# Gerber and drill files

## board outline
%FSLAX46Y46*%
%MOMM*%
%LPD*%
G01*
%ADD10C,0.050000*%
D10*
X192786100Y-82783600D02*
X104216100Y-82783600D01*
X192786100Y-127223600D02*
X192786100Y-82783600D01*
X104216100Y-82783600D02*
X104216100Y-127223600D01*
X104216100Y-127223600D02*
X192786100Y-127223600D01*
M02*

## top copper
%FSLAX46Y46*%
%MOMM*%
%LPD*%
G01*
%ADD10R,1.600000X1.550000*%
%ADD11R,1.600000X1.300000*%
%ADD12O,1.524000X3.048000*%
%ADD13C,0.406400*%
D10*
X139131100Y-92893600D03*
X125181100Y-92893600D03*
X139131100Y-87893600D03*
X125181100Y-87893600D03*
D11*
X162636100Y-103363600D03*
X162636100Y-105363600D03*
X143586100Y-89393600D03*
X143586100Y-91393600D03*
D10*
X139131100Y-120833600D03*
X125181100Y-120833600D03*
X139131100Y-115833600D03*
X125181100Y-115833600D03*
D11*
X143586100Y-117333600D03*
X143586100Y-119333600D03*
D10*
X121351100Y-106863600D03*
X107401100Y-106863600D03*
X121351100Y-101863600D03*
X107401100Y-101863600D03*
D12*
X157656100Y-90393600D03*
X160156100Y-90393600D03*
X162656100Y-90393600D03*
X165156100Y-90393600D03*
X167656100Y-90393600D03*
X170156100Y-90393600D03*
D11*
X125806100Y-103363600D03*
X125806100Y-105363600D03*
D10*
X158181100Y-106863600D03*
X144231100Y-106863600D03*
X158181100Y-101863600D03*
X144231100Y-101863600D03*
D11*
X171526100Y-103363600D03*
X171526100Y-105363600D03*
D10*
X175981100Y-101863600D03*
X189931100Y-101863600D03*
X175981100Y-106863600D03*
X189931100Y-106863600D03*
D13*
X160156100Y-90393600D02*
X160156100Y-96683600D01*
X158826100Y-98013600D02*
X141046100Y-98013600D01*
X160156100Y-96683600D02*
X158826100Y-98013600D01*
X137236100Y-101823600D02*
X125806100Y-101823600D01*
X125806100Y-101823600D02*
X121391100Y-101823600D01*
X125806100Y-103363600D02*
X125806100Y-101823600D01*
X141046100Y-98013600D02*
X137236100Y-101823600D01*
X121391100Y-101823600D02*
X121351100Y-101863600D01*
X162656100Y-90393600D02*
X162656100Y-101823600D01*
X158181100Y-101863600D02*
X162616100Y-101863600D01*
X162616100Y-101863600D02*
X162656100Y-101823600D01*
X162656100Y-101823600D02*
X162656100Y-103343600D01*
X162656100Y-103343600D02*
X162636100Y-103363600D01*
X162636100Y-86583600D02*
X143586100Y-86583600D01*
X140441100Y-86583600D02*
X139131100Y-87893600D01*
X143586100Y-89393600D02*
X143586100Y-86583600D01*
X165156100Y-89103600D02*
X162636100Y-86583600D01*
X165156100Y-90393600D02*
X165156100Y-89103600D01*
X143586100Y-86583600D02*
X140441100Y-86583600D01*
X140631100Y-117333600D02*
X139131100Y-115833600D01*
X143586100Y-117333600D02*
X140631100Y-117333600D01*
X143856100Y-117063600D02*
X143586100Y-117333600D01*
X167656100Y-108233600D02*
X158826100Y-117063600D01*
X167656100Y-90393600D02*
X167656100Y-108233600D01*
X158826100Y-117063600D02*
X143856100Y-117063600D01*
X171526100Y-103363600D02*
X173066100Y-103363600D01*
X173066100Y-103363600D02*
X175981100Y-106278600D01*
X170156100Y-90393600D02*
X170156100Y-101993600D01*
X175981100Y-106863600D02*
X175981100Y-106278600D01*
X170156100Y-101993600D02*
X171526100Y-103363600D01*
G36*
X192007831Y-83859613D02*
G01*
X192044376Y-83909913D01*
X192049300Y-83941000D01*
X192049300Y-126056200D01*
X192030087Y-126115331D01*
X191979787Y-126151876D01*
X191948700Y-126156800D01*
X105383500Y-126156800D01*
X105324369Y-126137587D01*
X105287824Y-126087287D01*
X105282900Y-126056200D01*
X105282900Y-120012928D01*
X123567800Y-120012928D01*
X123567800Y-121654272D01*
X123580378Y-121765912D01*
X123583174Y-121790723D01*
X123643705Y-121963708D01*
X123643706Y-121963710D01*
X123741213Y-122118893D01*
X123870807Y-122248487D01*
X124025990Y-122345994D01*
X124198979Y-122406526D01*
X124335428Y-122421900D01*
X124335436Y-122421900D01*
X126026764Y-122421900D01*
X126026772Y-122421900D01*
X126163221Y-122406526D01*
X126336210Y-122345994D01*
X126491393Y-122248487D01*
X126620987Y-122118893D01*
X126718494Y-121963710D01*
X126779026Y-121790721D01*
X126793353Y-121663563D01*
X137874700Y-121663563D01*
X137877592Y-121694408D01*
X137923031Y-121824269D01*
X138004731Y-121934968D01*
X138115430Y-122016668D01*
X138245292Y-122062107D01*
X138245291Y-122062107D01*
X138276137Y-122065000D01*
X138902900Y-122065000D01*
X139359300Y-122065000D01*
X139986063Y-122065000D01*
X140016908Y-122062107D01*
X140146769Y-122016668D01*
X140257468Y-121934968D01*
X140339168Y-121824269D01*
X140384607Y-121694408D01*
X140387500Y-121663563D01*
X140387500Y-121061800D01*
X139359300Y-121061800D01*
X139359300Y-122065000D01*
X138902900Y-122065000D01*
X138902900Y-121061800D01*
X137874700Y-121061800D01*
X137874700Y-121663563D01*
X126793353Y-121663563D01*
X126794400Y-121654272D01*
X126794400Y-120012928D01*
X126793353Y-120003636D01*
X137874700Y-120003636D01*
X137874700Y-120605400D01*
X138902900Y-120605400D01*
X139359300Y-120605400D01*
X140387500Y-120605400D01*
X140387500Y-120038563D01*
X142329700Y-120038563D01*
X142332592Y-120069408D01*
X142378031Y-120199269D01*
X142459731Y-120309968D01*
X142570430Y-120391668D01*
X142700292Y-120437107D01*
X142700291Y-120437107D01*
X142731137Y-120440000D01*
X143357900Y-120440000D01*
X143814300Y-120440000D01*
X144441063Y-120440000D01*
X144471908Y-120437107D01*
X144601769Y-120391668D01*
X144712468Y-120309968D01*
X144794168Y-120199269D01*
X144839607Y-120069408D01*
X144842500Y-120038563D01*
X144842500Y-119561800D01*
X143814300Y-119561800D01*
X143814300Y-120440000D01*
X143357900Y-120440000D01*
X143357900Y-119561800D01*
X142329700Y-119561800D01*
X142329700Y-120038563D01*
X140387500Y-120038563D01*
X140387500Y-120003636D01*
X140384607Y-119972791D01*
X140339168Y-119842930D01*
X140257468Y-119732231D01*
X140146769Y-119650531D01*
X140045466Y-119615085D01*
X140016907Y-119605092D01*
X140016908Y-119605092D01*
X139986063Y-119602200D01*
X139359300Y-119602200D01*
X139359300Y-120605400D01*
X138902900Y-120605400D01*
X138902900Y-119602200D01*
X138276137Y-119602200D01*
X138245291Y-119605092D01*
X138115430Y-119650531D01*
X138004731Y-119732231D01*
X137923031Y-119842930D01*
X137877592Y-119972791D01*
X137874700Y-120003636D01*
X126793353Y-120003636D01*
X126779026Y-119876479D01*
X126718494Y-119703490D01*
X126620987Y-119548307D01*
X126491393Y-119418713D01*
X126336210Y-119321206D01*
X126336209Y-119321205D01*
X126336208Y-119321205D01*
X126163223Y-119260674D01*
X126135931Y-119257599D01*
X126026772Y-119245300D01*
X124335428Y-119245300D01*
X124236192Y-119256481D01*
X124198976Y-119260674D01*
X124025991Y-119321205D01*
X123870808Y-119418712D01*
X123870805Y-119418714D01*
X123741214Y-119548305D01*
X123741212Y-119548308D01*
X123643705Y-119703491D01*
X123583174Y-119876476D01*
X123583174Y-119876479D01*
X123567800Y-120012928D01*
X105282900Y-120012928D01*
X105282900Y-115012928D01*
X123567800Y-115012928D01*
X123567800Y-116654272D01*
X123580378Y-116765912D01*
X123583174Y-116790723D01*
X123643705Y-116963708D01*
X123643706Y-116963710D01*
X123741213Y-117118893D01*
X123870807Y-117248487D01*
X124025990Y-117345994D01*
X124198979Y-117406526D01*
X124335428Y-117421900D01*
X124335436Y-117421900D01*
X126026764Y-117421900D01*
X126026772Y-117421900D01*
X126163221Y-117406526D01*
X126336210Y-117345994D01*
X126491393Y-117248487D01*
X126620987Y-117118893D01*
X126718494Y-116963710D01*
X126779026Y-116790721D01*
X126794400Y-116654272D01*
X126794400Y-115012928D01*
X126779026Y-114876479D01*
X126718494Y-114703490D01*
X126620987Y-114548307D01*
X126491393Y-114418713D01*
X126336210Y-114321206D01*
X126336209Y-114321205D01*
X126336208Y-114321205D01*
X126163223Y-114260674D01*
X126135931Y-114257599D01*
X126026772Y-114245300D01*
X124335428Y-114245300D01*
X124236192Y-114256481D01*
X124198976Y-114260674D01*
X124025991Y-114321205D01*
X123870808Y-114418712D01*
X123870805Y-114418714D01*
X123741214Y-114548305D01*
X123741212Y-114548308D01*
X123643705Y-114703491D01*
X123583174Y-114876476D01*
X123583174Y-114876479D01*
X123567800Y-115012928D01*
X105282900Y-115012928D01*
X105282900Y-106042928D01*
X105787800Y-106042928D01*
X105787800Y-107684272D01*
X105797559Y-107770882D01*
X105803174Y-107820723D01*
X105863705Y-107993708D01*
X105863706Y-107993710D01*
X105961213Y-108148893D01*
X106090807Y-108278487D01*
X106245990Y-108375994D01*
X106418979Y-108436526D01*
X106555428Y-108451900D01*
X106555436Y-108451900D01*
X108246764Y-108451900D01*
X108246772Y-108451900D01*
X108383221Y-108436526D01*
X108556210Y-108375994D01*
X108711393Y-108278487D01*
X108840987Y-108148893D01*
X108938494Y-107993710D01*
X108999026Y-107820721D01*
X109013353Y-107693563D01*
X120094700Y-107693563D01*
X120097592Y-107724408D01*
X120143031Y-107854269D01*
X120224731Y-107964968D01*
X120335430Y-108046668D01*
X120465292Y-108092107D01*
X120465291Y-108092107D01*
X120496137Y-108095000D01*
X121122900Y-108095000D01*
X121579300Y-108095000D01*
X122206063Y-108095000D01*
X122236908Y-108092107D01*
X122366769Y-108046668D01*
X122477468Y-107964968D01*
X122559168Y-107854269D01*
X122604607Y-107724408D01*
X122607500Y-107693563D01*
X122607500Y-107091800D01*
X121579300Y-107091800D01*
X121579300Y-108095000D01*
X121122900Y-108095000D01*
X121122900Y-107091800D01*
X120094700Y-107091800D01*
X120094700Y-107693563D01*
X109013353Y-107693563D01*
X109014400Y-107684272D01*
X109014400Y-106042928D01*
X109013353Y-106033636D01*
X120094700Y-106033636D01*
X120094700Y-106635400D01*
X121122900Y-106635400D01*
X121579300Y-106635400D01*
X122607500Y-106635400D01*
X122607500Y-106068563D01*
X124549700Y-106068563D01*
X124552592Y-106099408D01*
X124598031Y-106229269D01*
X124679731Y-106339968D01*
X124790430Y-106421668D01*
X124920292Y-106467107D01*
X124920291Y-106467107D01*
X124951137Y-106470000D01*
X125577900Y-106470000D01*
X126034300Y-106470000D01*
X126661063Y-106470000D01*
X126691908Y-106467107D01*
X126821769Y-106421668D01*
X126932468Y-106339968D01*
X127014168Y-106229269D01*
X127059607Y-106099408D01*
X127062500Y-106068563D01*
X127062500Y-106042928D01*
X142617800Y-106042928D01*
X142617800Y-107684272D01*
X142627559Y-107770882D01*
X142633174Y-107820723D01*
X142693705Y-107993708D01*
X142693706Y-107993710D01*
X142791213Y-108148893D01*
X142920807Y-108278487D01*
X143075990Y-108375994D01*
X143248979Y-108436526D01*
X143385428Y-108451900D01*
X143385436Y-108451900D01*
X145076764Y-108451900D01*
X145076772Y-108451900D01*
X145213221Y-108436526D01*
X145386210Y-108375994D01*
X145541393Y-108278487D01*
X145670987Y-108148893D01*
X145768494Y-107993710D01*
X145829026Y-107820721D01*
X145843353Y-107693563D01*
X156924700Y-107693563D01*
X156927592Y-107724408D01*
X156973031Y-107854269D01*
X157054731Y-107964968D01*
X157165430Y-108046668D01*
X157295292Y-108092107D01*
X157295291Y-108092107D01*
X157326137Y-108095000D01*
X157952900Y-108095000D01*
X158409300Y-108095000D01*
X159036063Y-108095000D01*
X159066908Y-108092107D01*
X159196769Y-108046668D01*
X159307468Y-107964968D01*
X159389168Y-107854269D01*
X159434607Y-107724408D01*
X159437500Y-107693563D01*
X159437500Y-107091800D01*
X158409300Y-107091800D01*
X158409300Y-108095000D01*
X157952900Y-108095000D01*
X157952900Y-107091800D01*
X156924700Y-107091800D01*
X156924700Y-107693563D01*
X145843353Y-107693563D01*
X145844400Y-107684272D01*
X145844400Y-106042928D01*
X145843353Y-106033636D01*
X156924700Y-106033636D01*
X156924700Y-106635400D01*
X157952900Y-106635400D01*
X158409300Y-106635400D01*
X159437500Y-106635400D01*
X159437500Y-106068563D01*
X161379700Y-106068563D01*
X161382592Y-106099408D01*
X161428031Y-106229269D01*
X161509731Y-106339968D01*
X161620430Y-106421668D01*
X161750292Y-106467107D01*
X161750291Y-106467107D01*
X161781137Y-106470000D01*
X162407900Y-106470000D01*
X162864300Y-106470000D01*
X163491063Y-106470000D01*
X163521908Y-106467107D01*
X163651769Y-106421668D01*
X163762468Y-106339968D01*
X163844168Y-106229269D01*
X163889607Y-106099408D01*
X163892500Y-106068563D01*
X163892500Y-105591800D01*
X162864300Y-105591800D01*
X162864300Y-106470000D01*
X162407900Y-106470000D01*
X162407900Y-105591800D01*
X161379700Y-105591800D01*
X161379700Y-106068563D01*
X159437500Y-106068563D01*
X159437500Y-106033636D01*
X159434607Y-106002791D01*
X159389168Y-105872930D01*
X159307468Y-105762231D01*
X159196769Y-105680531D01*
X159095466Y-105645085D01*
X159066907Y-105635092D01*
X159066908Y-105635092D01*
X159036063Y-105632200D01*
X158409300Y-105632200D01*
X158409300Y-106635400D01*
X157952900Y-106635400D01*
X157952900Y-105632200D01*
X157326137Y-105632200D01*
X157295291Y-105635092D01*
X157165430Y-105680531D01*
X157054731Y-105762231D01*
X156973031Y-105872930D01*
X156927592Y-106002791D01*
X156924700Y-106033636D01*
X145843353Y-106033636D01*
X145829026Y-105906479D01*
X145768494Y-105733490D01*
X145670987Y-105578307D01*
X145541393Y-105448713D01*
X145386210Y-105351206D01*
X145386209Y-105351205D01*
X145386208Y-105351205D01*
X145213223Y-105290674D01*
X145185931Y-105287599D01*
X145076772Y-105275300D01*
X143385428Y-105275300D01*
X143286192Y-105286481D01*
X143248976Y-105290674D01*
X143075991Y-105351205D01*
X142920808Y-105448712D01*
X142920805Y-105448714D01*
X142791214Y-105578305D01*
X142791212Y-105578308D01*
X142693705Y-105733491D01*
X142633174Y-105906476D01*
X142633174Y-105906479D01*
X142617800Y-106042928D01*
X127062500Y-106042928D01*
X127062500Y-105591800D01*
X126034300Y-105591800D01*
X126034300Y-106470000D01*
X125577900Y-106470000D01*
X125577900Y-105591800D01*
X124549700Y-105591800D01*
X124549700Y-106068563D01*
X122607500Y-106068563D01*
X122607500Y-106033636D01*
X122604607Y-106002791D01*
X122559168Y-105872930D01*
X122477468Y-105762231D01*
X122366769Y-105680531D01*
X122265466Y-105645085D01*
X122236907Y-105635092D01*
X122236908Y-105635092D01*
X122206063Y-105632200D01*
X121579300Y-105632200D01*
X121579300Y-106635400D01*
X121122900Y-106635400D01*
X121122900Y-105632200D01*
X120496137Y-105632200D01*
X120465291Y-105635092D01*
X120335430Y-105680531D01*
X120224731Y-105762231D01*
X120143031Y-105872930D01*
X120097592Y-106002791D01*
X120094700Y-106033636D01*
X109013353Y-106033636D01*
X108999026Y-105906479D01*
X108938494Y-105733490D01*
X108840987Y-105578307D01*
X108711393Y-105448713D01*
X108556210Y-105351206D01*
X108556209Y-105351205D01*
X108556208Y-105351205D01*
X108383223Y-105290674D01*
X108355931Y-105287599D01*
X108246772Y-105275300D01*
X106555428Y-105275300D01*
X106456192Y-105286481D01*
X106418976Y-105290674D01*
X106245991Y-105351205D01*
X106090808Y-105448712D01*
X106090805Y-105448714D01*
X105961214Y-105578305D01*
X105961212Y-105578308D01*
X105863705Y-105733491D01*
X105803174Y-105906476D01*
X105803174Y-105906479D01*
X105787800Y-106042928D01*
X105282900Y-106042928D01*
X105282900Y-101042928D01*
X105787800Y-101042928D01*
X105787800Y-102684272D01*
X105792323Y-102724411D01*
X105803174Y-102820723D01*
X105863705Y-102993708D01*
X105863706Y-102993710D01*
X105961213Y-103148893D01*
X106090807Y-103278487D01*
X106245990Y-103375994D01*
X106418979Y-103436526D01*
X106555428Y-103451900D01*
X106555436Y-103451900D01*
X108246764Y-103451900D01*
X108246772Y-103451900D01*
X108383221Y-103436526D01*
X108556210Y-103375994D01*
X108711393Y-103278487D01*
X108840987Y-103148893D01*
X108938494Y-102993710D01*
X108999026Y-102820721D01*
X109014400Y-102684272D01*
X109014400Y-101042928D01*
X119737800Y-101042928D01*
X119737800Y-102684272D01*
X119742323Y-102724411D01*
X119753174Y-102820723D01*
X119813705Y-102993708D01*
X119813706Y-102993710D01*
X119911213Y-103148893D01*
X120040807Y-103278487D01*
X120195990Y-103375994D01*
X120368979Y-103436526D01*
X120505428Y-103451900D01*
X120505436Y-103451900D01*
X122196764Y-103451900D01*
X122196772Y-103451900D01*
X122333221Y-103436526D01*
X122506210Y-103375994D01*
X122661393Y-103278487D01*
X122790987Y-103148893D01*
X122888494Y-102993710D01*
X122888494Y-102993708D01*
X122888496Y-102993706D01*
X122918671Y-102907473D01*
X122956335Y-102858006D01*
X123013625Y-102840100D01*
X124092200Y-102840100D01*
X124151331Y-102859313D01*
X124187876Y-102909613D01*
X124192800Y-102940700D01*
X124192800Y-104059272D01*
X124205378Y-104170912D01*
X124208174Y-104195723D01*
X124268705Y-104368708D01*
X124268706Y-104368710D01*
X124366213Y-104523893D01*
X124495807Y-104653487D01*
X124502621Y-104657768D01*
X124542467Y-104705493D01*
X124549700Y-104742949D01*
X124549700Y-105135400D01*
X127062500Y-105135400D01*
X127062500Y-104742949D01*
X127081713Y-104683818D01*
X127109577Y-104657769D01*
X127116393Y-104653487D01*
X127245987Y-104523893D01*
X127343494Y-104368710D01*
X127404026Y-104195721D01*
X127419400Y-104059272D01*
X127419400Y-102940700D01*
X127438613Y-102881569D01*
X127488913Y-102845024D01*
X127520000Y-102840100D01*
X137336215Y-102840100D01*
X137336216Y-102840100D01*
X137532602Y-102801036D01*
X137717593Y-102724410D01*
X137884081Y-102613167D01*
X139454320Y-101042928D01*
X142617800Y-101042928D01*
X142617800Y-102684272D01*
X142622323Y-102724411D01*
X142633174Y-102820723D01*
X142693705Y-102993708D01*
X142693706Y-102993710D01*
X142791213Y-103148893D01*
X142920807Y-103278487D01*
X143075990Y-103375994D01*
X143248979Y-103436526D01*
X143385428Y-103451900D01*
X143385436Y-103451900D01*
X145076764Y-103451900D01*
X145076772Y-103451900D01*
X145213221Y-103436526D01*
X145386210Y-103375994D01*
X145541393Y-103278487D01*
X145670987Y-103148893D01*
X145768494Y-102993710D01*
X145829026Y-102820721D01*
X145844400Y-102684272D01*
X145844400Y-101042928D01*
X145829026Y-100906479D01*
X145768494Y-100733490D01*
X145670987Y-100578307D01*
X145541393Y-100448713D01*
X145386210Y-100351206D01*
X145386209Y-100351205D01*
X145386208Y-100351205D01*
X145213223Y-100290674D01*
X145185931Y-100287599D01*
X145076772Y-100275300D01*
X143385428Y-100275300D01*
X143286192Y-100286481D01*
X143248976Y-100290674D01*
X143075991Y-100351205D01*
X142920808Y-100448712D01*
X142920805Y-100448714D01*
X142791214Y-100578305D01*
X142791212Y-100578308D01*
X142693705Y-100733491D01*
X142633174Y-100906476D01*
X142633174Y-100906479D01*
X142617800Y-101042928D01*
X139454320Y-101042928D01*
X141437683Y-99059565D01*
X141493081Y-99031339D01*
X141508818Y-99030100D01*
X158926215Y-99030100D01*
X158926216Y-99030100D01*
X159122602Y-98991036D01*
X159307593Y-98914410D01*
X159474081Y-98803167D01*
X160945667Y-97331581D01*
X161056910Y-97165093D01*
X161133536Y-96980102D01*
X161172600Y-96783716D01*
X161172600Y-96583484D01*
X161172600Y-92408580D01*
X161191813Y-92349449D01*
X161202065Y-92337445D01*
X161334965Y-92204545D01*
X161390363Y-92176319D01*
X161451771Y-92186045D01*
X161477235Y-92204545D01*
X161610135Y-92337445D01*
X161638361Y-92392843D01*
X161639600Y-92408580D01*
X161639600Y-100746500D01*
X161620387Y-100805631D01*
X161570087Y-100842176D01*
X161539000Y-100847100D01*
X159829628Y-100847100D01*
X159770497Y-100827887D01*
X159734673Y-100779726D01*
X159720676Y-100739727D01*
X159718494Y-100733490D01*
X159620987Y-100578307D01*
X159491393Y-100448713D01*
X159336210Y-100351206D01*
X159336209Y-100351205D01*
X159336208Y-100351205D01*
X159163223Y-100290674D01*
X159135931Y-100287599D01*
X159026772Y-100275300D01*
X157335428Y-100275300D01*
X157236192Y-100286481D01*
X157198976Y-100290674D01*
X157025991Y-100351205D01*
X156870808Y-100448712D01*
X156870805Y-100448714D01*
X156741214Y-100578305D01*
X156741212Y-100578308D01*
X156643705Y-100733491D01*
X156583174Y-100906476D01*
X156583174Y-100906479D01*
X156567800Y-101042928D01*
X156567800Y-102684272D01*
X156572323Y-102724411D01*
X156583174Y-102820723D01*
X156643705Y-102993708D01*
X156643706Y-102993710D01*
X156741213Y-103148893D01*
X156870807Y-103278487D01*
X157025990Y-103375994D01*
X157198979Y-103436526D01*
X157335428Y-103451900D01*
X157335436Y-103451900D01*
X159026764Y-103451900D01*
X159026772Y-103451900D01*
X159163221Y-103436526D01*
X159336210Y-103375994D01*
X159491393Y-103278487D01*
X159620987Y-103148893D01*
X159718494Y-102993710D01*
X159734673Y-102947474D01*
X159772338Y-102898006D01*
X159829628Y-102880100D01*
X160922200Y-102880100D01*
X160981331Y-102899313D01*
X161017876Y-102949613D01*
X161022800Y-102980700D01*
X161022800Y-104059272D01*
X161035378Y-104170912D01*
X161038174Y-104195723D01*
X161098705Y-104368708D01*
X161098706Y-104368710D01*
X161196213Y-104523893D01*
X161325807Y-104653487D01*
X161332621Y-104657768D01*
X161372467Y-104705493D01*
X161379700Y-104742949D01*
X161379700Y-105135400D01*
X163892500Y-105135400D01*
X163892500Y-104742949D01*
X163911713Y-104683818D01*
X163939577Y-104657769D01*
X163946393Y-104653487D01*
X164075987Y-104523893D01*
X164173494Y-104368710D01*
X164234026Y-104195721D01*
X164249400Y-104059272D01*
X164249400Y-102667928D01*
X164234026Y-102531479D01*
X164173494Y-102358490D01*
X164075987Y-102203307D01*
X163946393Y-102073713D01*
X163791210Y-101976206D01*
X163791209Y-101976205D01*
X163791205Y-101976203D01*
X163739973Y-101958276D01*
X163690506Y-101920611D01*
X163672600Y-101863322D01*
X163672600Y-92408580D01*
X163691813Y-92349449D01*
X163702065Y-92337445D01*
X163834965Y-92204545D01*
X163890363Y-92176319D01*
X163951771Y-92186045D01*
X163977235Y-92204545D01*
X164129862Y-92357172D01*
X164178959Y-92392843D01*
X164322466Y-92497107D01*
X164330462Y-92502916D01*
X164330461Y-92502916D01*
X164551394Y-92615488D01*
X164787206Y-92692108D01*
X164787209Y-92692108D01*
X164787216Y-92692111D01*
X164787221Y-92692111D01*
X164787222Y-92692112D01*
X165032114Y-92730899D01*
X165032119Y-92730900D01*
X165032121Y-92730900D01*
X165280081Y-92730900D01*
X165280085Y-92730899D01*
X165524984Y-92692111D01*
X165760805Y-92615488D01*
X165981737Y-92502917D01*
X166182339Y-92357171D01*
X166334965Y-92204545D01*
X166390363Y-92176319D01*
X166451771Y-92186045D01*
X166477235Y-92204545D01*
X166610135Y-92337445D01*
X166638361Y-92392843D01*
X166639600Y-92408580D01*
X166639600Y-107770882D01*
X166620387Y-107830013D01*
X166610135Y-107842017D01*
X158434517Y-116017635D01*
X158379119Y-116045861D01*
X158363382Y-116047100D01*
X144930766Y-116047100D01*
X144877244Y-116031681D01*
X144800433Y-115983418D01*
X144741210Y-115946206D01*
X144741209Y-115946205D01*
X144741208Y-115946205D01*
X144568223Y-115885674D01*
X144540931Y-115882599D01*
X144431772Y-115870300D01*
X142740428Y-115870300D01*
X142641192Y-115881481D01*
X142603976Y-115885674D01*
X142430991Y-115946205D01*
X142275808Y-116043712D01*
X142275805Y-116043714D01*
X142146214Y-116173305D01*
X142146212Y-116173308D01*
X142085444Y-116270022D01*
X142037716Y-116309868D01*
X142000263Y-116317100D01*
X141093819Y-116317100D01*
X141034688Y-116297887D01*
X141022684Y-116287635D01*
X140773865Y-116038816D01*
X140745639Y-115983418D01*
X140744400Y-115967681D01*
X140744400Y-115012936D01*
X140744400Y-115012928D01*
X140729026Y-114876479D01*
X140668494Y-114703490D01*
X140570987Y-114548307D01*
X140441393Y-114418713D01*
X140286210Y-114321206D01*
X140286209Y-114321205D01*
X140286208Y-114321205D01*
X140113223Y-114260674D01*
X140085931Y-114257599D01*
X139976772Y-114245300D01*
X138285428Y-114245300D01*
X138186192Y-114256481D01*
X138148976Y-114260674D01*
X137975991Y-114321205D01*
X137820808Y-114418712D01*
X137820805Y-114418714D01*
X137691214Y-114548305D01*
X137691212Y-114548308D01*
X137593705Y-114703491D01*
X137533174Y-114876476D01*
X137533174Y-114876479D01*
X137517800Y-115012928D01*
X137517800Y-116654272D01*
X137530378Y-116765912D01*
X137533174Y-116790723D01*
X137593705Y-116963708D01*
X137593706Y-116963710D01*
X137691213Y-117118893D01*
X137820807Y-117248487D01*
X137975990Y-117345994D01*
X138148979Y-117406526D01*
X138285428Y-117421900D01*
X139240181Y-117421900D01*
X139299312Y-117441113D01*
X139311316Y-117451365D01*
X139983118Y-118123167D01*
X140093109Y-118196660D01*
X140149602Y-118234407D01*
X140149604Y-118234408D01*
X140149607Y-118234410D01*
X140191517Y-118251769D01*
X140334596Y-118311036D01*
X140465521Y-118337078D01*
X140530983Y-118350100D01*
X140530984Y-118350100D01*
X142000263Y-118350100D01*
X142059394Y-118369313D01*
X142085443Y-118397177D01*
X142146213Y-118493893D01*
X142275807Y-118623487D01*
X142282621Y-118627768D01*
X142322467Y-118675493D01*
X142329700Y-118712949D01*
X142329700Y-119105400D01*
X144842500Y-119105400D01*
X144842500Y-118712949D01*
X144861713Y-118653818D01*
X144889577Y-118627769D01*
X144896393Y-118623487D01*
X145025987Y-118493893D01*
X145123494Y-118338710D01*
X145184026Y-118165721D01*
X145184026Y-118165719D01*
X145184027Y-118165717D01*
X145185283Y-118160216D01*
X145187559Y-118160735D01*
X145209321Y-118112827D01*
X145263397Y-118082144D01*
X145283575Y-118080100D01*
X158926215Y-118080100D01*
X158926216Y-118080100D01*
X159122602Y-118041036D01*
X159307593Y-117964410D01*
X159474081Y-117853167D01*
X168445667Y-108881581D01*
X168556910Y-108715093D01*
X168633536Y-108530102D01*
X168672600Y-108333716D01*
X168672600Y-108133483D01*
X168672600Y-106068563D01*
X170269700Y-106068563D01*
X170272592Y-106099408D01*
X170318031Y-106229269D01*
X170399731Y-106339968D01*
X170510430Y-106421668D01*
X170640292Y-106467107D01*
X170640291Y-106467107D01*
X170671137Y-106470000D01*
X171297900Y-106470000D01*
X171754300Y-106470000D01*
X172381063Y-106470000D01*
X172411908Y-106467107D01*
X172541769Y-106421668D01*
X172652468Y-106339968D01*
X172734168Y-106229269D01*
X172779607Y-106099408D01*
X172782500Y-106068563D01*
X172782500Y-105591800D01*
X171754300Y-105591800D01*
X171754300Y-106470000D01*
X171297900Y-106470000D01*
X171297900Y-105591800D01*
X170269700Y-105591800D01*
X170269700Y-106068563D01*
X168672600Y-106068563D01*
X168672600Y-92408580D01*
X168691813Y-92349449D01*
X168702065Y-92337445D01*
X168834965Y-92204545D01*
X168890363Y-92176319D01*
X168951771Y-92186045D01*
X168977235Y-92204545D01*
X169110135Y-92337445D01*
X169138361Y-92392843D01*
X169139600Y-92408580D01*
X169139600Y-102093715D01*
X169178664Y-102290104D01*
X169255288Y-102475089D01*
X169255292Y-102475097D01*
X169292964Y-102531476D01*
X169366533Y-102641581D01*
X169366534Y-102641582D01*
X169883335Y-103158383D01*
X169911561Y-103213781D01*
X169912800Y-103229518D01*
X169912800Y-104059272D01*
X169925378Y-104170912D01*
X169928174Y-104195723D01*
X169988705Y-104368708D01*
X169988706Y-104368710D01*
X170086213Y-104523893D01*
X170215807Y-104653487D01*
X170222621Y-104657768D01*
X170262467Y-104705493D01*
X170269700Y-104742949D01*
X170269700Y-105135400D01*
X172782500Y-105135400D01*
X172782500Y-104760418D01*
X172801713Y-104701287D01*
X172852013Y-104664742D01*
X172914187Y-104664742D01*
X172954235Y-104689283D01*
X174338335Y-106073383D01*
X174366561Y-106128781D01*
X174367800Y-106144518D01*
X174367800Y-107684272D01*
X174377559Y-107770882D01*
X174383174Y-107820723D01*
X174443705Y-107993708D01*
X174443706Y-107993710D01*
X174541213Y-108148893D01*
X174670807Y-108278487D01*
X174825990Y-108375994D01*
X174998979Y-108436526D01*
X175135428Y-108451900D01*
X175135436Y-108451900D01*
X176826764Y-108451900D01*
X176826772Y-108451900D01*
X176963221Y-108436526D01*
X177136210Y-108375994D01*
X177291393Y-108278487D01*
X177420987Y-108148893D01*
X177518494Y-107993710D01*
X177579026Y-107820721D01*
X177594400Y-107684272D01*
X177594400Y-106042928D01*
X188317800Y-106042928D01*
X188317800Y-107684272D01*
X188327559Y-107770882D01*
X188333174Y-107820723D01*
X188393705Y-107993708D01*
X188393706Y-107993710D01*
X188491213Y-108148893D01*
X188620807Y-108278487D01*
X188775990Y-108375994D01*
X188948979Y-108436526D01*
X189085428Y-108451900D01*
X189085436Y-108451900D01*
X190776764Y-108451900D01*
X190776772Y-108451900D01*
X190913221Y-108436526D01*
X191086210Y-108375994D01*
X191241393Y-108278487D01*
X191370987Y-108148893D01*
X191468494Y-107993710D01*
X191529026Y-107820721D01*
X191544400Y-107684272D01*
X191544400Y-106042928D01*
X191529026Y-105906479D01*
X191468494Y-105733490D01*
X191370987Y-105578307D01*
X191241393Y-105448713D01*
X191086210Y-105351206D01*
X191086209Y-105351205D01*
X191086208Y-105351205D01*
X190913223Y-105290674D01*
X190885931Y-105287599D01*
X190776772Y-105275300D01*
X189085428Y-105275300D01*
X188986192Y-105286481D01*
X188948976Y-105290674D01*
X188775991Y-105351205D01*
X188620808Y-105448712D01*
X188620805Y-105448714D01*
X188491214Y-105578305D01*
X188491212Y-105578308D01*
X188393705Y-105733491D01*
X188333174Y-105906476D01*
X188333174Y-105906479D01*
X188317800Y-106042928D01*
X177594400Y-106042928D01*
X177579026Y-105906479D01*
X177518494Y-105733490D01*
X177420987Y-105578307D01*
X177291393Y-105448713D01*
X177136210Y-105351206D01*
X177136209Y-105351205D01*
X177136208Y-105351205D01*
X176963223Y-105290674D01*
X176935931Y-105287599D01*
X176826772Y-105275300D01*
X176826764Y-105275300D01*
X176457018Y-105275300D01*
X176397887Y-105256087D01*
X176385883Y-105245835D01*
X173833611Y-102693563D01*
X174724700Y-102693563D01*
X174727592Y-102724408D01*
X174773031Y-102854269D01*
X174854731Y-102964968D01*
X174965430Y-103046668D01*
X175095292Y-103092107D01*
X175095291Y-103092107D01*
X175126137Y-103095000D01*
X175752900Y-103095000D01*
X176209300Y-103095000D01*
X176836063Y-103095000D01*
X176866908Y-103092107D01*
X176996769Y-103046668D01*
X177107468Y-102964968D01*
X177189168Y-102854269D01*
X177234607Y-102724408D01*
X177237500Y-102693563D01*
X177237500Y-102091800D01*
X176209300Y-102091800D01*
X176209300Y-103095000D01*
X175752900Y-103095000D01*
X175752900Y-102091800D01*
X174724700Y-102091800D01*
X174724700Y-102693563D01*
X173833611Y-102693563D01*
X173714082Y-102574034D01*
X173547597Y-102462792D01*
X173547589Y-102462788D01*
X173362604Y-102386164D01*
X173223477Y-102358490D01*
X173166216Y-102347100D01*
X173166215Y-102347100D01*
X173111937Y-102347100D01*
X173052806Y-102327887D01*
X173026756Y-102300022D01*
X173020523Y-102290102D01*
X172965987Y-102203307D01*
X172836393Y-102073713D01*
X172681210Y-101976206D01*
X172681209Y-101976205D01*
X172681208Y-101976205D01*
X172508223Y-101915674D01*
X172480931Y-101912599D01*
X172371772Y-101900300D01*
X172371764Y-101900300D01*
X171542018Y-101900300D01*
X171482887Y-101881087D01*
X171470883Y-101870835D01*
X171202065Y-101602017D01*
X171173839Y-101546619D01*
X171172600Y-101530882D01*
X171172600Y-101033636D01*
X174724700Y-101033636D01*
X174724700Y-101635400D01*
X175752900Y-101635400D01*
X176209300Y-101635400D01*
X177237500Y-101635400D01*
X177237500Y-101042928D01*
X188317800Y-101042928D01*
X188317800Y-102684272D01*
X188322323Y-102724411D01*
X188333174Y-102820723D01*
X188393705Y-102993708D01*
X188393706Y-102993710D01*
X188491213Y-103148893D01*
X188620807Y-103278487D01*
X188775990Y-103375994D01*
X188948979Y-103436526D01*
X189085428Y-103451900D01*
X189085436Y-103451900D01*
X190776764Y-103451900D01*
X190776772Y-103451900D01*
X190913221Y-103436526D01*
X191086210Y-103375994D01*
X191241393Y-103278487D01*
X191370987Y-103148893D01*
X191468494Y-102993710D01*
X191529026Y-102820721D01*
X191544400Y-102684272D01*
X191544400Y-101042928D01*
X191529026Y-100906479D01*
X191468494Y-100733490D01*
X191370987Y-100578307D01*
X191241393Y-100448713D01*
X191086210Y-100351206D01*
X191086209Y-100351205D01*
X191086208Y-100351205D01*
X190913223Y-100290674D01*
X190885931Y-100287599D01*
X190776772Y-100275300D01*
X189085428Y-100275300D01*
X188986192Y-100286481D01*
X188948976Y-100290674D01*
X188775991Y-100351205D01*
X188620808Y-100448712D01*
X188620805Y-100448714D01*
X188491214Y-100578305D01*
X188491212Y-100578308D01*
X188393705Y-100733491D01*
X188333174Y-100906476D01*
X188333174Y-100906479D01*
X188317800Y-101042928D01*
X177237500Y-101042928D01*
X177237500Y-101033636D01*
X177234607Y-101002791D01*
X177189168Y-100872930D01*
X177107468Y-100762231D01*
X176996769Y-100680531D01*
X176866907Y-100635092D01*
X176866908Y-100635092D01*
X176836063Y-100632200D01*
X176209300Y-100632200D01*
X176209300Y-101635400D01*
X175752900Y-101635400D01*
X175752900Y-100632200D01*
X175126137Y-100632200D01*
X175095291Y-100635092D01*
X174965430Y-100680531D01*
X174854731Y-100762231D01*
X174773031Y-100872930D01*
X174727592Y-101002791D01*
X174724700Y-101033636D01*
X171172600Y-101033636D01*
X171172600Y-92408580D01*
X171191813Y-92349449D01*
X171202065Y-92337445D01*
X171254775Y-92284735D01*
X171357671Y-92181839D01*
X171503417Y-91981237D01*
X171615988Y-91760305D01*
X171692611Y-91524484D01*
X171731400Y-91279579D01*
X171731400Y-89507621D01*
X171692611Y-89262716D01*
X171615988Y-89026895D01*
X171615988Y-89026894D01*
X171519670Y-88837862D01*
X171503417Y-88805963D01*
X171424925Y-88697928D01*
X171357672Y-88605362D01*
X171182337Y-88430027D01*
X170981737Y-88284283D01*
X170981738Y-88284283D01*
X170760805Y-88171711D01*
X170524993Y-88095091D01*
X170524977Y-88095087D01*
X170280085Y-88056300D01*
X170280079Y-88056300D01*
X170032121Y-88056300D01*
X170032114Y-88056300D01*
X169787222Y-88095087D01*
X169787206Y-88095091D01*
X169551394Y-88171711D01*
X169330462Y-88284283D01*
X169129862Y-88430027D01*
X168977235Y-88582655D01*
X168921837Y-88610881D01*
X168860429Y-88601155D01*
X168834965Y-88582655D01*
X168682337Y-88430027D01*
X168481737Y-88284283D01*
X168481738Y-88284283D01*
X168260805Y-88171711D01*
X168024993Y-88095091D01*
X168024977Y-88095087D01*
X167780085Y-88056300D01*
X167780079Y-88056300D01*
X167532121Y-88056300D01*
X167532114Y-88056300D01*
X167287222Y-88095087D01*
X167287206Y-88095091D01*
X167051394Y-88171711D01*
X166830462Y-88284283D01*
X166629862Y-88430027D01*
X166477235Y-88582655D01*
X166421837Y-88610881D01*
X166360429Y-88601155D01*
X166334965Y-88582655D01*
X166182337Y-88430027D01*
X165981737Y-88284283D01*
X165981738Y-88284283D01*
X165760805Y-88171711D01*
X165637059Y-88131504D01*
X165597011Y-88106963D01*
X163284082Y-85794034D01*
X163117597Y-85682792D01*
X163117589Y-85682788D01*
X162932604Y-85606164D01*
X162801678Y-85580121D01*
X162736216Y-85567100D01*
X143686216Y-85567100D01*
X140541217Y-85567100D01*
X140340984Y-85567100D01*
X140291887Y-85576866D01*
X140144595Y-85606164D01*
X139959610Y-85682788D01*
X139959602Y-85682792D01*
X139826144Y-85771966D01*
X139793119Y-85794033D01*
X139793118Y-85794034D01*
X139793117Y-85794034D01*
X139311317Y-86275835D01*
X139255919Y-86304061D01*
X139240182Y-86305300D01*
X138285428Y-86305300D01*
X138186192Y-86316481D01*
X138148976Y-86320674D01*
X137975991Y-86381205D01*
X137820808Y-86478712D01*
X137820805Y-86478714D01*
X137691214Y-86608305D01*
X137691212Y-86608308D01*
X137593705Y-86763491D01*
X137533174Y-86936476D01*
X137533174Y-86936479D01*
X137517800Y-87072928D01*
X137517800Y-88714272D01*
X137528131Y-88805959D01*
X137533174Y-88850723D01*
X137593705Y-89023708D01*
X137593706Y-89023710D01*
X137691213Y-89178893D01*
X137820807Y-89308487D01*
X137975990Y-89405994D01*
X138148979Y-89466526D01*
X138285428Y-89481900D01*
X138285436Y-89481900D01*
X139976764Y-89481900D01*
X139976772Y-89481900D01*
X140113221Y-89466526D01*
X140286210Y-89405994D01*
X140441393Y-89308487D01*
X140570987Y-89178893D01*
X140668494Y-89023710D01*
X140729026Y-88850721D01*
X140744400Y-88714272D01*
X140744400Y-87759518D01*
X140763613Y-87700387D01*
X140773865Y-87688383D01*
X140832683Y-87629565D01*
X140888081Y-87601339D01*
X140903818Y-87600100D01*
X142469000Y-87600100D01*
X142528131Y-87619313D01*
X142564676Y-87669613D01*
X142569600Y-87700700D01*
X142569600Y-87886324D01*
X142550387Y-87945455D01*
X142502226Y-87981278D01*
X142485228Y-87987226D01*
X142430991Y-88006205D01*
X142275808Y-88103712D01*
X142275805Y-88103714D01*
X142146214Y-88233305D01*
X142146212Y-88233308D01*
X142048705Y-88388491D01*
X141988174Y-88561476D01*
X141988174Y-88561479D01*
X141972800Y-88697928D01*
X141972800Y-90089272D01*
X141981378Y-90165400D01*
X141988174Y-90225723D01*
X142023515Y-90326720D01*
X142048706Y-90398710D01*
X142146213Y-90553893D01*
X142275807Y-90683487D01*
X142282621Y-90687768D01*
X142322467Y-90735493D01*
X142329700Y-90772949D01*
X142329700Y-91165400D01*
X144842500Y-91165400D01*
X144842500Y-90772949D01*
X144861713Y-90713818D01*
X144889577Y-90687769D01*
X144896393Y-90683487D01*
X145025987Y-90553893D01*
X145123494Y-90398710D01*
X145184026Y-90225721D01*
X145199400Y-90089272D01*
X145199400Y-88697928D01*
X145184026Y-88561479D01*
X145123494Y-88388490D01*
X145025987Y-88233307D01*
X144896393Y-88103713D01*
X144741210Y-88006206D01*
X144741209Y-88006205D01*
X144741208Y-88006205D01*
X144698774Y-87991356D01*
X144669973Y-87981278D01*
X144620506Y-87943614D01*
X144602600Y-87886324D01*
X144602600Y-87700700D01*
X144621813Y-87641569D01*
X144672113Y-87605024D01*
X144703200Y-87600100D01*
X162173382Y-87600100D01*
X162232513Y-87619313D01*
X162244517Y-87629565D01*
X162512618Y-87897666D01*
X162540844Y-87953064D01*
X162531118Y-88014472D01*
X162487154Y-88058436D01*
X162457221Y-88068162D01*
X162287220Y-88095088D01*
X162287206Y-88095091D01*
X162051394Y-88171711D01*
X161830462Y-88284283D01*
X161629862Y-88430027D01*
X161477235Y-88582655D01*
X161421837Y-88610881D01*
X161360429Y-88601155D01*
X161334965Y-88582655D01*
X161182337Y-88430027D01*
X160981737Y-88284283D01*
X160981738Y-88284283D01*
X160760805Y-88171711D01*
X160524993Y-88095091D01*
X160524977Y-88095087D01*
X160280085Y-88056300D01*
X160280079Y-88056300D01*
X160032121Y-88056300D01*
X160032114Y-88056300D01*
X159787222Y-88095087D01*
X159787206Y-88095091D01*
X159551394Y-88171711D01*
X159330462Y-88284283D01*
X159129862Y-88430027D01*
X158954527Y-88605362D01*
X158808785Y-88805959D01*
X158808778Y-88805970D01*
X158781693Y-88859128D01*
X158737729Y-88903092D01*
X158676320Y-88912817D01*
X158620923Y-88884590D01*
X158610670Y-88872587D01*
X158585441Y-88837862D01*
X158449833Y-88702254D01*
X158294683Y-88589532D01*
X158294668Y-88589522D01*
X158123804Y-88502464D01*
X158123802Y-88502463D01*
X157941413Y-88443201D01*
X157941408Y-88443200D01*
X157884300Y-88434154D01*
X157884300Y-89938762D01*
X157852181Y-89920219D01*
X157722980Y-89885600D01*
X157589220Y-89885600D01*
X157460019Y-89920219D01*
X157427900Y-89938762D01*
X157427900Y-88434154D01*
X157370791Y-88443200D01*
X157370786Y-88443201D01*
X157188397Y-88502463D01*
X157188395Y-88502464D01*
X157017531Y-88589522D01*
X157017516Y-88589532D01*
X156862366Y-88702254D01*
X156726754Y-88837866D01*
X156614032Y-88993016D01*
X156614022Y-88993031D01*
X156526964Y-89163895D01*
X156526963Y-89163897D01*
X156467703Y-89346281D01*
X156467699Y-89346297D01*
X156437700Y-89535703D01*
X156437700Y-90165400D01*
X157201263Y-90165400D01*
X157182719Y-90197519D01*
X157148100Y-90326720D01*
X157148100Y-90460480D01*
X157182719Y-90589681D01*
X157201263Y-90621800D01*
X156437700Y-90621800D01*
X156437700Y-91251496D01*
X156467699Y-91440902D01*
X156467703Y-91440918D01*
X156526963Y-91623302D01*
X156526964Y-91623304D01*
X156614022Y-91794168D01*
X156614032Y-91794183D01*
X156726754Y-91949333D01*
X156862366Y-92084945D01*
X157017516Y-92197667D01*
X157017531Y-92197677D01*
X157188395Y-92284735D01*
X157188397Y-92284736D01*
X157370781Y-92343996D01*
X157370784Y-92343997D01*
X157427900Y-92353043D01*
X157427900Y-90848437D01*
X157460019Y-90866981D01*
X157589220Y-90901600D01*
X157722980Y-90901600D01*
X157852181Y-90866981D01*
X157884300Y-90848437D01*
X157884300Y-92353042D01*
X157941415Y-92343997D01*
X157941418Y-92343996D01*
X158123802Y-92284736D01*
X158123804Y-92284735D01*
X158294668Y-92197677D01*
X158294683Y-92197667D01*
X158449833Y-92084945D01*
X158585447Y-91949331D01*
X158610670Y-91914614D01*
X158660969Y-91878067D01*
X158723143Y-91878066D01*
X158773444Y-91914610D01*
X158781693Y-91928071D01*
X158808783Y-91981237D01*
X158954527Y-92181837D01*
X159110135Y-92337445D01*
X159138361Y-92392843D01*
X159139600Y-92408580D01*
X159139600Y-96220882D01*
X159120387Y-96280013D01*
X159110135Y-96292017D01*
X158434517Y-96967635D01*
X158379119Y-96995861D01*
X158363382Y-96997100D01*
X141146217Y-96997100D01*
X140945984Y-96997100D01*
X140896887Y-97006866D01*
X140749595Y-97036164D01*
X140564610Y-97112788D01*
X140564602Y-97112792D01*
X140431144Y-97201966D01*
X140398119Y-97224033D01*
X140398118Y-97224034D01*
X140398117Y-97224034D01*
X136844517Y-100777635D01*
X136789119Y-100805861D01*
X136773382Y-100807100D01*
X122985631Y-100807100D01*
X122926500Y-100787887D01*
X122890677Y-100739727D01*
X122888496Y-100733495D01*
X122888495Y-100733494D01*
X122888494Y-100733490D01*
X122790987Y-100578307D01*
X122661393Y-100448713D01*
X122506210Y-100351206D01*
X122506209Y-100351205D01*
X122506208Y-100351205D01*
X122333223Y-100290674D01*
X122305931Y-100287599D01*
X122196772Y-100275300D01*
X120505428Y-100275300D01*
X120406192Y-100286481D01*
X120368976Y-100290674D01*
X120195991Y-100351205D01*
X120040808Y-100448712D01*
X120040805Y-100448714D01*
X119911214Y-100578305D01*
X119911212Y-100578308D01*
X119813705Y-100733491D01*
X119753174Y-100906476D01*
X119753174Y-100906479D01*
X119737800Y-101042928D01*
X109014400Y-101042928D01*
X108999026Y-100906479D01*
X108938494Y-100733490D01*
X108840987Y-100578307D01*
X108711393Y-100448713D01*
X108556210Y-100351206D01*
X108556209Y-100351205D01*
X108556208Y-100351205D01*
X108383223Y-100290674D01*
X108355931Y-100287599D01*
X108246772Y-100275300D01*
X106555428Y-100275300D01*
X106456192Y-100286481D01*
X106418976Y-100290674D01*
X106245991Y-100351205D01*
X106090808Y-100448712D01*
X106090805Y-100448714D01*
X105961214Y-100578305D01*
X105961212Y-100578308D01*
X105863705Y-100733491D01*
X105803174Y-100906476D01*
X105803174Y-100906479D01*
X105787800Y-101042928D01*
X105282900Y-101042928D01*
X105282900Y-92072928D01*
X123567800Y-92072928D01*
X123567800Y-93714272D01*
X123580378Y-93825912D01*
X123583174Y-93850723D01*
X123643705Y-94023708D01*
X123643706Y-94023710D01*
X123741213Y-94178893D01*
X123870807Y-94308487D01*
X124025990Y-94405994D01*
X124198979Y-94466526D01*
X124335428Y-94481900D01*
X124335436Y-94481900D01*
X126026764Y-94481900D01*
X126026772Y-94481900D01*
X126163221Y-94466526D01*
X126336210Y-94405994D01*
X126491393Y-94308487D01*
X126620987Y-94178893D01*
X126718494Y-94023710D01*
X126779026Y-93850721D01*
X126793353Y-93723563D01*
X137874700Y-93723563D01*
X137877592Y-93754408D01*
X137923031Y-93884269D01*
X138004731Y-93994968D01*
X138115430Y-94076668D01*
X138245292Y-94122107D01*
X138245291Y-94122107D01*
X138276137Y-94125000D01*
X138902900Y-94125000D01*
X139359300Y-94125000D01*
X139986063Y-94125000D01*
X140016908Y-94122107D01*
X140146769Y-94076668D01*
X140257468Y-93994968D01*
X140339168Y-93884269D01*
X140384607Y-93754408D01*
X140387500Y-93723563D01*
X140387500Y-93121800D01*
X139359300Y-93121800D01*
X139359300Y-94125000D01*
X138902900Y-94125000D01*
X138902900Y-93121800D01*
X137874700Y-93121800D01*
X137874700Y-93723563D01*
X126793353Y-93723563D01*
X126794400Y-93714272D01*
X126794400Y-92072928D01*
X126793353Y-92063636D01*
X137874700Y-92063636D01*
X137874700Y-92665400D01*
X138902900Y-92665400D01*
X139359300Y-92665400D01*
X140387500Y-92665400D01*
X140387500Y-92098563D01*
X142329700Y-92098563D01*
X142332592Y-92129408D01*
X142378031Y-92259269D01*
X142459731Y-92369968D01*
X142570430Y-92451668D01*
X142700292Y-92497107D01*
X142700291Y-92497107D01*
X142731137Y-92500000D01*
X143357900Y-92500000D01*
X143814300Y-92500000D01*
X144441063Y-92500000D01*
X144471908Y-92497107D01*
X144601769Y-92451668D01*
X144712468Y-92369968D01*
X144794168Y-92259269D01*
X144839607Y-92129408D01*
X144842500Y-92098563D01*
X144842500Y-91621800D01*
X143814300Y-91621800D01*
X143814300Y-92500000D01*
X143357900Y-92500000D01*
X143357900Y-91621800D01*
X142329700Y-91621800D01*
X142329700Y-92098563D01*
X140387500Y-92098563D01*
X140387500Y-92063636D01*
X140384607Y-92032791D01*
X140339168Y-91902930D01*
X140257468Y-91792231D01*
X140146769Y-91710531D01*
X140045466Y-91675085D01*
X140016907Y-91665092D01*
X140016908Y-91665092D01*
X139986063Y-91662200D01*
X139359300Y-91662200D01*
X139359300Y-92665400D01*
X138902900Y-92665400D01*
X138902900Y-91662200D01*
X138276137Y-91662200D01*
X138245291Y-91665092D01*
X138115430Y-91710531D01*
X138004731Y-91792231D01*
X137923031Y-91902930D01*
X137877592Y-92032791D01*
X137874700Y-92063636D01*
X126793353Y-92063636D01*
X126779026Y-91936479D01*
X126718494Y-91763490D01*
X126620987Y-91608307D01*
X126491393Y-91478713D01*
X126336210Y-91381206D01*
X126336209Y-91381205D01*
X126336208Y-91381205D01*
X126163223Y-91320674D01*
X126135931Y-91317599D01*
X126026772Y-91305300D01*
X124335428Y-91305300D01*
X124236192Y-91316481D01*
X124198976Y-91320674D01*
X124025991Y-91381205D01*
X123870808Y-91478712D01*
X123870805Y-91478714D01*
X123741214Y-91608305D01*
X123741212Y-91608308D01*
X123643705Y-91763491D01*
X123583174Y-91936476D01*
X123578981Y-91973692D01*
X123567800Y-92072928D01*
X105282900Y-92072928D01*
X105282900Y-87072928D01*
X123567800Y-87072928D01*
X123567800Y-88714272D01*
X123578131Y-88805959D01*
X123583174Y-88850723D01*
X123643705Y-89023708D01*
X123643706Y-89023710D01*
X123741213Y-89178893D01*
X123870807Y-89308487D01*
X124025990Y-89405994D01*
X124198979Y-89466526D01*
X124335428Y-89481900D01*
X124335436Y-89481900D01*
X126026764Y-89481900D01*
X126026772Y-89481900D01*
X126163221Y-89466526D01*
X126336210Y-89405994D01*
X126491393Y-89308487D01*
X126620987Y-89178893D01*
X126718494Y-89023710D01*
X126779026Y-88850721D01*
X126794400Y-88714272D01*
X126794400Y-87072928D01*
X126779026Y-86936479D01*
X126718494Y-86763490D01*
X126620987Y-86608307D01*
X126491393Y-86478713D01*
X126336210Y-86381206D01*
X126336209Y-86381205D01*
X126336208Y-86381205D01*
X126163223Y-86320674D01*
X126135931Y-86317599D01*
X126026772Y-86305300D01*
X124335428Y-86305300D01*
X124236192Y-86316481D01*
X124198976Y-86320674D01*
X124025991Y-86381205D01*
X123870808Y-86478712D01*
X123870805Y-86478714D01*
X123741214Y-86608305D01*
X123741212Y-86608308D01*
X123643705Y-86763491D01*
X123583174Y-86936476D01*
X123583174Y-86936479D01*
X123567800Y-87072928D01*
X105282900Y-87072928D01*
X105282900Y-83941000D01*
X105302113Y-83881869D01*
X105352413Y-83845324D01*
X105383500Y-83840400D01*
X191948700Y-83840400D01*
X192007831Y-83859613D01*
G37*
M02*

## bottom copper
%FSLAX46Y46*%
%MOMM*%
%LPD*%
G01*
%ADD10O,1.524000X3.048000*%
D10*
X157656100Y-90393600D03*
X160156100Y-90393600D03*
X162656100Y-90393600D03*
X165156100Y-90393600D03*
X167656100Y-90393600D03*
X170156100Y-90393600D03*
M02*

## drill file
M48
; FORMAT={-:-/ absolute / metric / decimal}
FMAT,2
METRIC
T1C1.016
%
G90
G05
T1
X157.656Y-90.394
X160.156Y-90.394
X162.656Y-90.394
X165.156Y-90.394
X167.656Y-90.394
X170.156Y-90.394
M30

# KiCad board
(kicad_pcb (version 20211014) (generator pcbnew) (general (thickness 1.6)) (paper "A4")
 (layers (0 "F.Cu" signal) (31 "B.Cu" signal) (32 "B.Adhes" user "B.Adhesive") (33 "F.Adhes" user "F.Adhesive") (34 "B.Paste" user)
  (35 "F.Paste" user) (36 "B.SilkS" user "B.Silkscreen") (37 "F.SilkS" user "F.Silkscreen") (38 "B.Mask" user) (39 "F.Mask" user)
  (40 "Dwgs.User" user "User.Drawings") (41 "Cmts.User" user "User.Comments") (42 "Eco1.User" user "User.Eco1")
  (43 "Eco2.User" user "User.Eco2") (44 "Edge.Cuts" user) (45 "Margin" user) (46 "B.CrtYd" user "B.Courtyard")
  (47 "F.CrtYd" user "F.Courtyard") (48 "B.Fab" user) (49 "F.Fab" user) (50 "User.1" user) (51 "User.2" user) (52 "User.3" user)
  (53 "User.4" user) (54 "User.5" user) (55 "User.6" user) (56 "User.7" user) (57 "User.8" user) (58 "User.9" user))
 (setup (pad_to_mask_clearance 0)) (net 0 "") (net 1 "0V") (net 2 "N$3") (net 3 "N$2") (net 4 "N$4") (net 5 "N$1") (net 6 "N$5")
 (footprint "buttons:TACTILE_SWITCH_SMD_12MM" (layer "F.Cu") (at 132.1561 90.3936)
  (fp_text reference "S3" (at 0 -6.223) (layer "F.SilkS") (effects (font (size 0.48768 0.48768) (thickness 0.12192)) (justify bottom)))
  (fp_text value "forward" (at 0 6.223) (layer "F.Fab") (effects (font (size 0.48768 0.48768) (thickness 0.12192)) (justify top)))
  (pad "1" smd rect (at 6.975 2.5) (size 1.6 1.55) (layers "F.Cu" "F.Paste" "F.Mask") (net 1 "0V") (solder_mask_margin 0.1016))
  (pad "2" smd rect (at -6.975 2.5) (size 1.6 1.55) (layers "F.Cu" "F.Paste" "F.Mask") (solder_mask_margin 0.1016))
  (pad "3" smd rect (at 6.975 -2.5) (size 1.6 1.55) (layers "F.Cu" "F.Paste" "F.Mask") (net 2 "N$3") (solder_mask_margin 0.1016))
  (pad "4" smd rect (at -6.975 -2.5) (size 1.6 1.55) (layers "F.Cu" "F.Paste" "F.Mask") (solder_mask_margin 0.1016)))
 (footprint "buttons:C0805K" (layer "F.Cu") (at 162.6361 104.3636 -90)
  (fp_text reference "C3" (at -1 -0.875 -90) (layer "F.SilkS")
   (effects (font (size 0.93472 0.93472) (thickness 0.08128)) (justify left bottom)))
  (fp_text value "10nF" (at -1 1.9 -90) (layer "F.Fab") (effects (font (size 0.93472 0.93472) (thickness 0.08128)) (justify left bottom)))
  (pad "1" smd rect (at -1 0 270) (size 1.3 1.6) (layers "F.Cu" "F.Paste" "F.Mask") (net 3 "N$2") (solder_mask_margin 0.1016))
  (pad "2" smd rect (at 1 0 270) (size 1.3 1.6) (layers "F.Cu" "F.Paste" "F.Mask") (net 1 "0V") (solder_mask_margin 0.1016)))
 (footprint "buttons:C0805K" (layer "F.Cu") (at 143.5861 90.3936 -90)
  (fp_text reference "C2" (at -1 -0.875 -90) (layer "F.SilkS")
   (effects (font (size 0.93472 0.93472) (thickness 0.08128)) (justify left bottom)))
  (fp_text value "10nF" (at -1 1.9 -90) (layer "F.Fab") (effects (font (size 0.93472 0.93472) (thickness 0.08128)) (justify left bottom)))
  (pad "1" smd rect (at -1 0 270) (size 1.3 1.6) (layers "F.Cu" "F.Paste" "F.Mask") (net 2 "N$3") (solder_mask_margin 0.1016))
  (pad "2" smd rect (at 1 0 270) (size 1.3 1.6) (layers "F.Cu" "F.Paste" "F.Mask") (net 1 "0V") (solder_mask_margin 0.1016)))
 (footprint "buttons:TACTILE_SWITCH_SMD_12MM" (layer "F.Cu") (at 132.1561 118.3336)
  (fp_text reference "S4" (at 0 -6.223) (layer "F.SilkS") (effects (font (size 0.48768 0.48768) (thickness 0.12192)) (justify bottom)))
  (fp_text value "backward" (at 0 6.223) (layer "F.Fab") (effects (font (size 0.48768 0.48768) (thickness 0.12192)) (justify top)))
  (pad "1" smd rect (at 6.975 2.5) (size 1.6 1.55) (layers "F.Cu" "F.Paste" "F.Mask") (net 1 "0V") (solder_mask_margin 0.1016))
  (pad "2" smd rect (at -6.975 2.5) (size 1.6 1.55) (layers "F.Cu" "F.Paste" "F.Mask") (solder_mask_margin 0.1016))
  (pad "3" smd rect (at 6.975 -2.5) (size 1.6 1.55) (layers "F.Cu" "F.Paste" "F.Mask") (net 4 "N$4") (solder_mask_margin 0.1016))
  (pad "4" smd rect (at -6.975 -2.5) (size 1.6 1.55) (layers "F.Cu" "F.Paste" "F.Mask") (solder_mask_margin 0.1016)))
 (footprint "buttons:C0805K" (layer "F.Cu") (at 143.5861 118.3336 -90)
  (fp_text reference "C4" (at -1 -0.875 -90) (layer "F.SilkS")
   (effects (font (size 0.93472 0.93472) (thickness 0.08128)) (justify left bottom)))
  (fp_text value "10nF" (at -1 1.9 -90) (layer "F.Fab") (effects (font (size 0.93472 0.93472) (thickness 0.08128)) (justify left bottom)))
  (pad "1" smd rect (at -1 0 270) (size 1.3 1.6) (layers "F.Cu" "F.Paste" "F.Mask") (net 4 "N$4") (solder_mask_margin 0.1016))
  (pad "2" smd rect (at 1 0 270) (size 1.3 1.6) (layers "F.Cu" "F.Paste" "F.Mask") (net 1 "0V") (solder_mask_margin 0.1016)))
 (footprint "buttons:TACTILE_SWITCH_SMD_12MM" (layer "F.Cu") (at 114.3761 104.3636)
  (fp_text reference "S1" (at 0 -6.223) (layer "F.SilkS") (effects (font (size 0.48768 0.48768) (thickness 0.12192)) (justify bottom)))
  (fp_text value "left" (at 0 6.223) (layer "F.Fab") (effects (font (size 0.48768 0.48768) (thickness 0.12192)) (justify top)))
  (pad "1" smd rect (at 6.975 2.5) (size 1.6 1.55) (layers "F.Cu" "F.Paste" "F.Mask") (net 1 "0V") (solder_mask_margin 0.1016))
  (pad "2" smd rect (at -6.975 2.5) (size 1.6 1.55) (layers "F.Cu" "F.Paste" "F.Mask") (solder_mask_margin 0.1016))
  (pad "3" smd rect (at 6.975 -2.5) (size 1.6 1.55) (layers "F.Cu" "F.Paste" "F.Mask") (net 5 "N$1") (solder_mask_margin 0.1016))
  (pad "4" smd rect (at -6.975 -2.5) (size 1.6 1.55) (layers "F.Cu" "F.Paste" "F.Mask") (solder_mask_margin 0.1016)))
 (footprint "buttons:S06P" (layer "F.Cu") (at 163.9061 90.3936 180)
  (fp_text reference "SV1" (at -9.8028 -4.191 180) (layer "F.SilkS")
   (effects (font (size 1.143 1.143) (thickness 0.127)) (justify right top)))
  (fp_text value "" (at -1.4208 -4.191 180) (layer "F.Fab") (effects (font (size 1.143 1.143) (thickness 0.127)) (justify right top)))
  (pad "1" thru_hole oval (at 6.25 0 270) (size 3.048 1.524) (drill 1.016) (layers *.Cu *.Mask) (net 1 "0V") (solder_mask_margin 0.1016))
  (pad "2" thru_hole oval (at 3.75 0 270) (size 3.048 1.524) (drill 1.016) (layers *.Cu *.Mask) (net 5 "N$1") (solder_mask_margin 0.1016))
  (pad "3" thru_hole oval (at 1.25 0 270) (size 3.048 1.524) (drill 1.016) (layers *.Cu *.Mask) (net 3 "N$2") (solder_mask_margin 0.1016))
  (pad "4" thru_hole oval (at -1.25 0 270) (size 3.048 1.524) (drill 1.016) (layers *.Cu *.Mask) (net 2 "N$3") (solder_mask_margin 0.1016))
  (pad "5" thru_hole oval (at -3.75 0 270) (size 3.048 1.524) (drill 1.016) (layers *.Cu *.Mask) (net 4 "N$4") (solder_mask_margin 0.1016))
  (pad "6" thru_hole oval (at -6.25 0 270) (size 3.048 1.524) (drill 1.016) (layers *.Cu *.Mask) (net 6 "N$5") (solder_mask_margin 0.1016)))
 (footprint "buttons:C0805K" (layer "F.Cu") (at 125.8061 104.3636 -90)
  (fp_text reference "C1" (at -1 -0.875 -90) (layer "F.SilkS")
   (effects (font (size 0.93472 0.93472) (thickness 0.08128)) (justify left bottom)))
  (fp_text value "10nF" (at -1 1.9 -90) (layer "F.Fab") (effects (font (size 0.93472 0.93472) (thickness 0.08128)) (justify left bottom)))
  (pad "1" smd rect (at -1 0 270) (size 1.3 1.6) (layers "F.Cu" "F.Paste" "F.Mask") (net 5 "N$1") (solder_mask_margin 0.1016))
  (pad "2" smd rect (at 1 0 270) (size 1.3 1.6) (layers "F.Cu" "F.Paste" "F.Mask") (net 1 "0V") (solder_mask_margin 0.1016)))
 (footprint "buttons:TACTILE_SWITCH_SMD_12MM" (layer "F.Cu") (at 151.2061 104.3636)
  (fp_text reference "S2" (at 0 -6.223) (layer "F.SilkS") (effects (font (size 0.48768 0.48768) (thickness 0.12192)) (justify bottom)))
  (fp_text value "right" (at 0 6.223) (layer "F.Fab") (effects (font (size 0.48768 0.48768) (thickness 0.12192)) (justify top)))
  (pad "1" smd rect (at 6.975 2.5) (size 1.6 1.55) (layers "F.Cu" "F.Paste" "F.Mask") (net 1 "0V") (solder_mask_margin 0.1016))
  (pad "2" smd rect (at -6.975 2.5) (size 1.6 1.55) (layers "F.Cu" "F.Paste" "F.Mask") (solder_mask_margin 0.1016))
  (pad "3" smd rect (at 6.975 -2.5) (size 1.6 1.55) (layers "F.Cu" "F.Paste" "F.Mask") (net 3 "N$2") (solder_mask_margin 0.1016))
  (pad "4" smd rect (at -6.975 -2.5) (size 1.6 1.55) (layers "F.Cu" "F.Paste" "F.Mask") (solder_mask_margin 0.1016)))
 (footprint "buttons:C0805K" (layer "F.Cu") (at 171.5261 104.3636 -90)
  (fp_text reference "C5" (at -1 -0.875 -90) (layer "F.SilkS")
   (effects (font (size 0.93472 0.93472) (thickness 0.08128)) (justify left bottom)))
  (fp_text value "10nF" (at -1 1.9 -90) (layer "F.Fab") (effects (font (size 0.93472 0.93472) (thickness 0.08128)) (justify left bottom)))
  (pad "1" smd rect (at -1 0 270) (size 1.3 1.6) (layers "F.Cu" "F.Paste" "F.Mask") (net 6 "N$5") (solder_mask_margin 0.1016))
  (pad "2" smd rect (at 1 0 270) (size 1.3 1.6) (layers "F.Cu" "F.Paste" "F.Mask") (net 1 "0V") (solder_mask_margin 0.1016)))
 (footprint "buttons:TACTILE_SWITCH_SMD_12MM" (layer "F.Cu") (at 182.9561 104.3636 180)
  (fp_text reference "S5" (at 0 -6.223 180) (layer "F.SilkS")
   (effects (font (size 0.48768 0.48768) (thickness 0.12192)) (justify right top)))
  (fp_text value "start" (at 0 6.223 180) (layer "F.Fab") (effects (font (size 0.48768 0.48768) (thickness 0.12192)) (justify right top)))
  (pad "1" smd rect (at 6.975 2.5 180) (size 1.6 1.55) (layers "F.Cu" "F.Paste" "F.Mask") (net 1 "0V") (solder_mask_margin 0.1016))
  (pad "2" smd rect (at -6.975 2.5 180) (size 1.6 1.55) (layers "F.Cu" "F.Paste" "F.Mask") (solder_mask_margin 0.1016))
  (pad "3" smd rect (at 6.975 -2.5 180) (size 1.6 1.55) (layers "F.Cu" "F.Paste" "F.Mask") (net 6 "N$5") (solder_mask_margin 0.1016))
  (pad "4" smd rect (at -6.975 -2.5 180) (size 1.6 1.55) (layers "F.Cu" "F.Paste" "F.Mask") (solder_mask_margin 0.1016)))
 (gr_line (start 192.7861 82.7836) (end 104.2161 82.7836) (layer "Edge.Cuts") (width 0.05))
 (gr_line (start 192.7861 127.2236) (end 192.7861 82.7836) (layer "Edge.Cuts") (width 0.05))
 (gr_line (start 104.2161 82.7836) (end 104.2161 127.2236) (layer "Edge.Cuts") (width 0.05))
 (gr_line (start 104.2161 127.2236) (end 192.7861 127.2236) (layer "Edge.Cuts") (width 0.05))
 (segment (start 160.1561 90.3936) (end 160.1561 96.6836) (width 0.4064) (layer "F.Cu") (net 5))
 (segment (start 158.8261 98.0136) (end 141.0461 98.0136) (width 0.4064) (layer "F.Cu") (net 5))
 (segment (start 160.1561 96.6836) (end 158.8261 98.0136) (width 0.4064) (layer "F.Cu") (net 5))
 (segment (start 137.2361 101.8236) (end 125.8061 101.8236) (width 0.4064) (layer "F.Cu") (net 5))
 (segment (start 125.8061 101.8236) (end 121.3911 101.8236) (width 0.4064) (layer "F.Cu") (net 5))
 (segment (start 125.8061 103.3636) (end 125.8061 101.8236) (width 0.4064) (layer "F.Cu") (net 5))
 (segment (start 141.0461 98.0136) (end 137.2361 101.8236) (width 0.4064) (layer "F.Cu") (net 5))
 (segment (start 121.3911 101.8236) (end 121.3511 101.8636) (width 0.4064) (layer "F.Cu") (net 5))
 (segment (start 162.6561 90.3936) (end 162.6561 101.8236) (width 0.4064) (layer "F.Cu") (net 3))
 (segment (start 158.1811 101.8636) (end 162.6161 101.8636) (width 0.4064) (layer "F.Cu") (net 3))
 (segment (start 162.6161 101.8636) (end 162.6561 101.8236) (width 0.4064) (layer "F.Cu") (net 3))
 (segment (start 162.6561 101.8236) (end 162.6561 103.3436) (width 0.4064) (layer "F.Cu") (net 3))
 (segment (start 162.6561 103.3436) (end 162.6361 103.3636) (width 0.4064) (layer "F.Cu") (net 3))
 (segment (start 162.6361 86.5836) (end 143.5861 86.5836) (width 0.4064) (layer "F.Cu") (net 2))
 (segment (start 140.4411 86.5836) (end 139.1311 87.8936) (width 0.4064) (layer "F.Cu") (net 2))
 (segment (start 143.5861 89.3936) (end 143.5861 86.5836) (width 0.4064) (layer "F.Cu") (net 2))
 (segment (start 165.1561 89.1036) (end 162.6361 86.5836) (width 0.4064) (layer "F.Cu") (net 2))
 (segment (start 165.1561 90.3936) (end 165.1561 89.1036) (width 0.4064) (layer "F.Cu") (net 2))
 (segment (start 143.5861 86.5836) (end 140.4411 86.5836) (width 0.4064) (layer "F.Cu") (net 2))
 (segment (start 140.6311 117.3336) (end 139.1311 115.8336) (width 0.4064) (layer "F.Cu") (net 4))
 (segment (start 143.5861 117.3336) (end 140.6311 117.3336) (width 0.4064) (layer "F.Cu") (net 4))
 (segment (start 143.8561 117.0636) (end 143.5861 117.3336) (width 0.4064) (layer "F.Cu") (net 4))
 (segment (start 167.6561 108.2336) (end 158.8261 117.0636) (width 0.4064) (layer "F.Cu") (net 4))
 (segment (start 167.6561 90.3936) (end 167.6561 108.2336) (width 0.4064) (layer "F.Cu") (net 4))
 (segment (start 158.8261 117.0636) (end 143.8561 117.0636) (width 0.4064) (layer "F.Cu") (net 4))
 (segment (start 171.5261 103.3636) (end 173.0661 103.3636) (width 0.4064) (layer "F.Cu") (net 6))
 (segment (start 173.0661 103.3636) (end 175.9811 106.2786) (width 0.4064) (layer "F.Cu") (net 6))
 (segment (start 170.1561 90.3936) (end 170.1561 101.9936) (width 0.4064) (layer "F.Cu") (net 6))
 (segment (start 175.9811 106.8636) (end 175.9811 106.2786) (width 0.4064) (layer "F.Cu") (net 6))
 (segment (start 170.1561 101.9936) (end 171.5261 103.3636) (width 0.4064) (layer "F.Cu") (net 6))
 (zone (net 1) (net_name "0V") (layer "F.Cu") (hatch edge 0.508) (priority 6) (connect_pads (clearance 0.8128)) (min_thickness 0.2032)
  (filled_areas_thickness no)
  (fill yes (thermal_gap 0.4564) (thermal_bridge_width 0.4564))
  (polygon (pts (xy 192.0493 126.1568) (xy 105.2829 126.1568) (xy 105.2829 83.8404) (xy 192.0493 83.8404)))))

